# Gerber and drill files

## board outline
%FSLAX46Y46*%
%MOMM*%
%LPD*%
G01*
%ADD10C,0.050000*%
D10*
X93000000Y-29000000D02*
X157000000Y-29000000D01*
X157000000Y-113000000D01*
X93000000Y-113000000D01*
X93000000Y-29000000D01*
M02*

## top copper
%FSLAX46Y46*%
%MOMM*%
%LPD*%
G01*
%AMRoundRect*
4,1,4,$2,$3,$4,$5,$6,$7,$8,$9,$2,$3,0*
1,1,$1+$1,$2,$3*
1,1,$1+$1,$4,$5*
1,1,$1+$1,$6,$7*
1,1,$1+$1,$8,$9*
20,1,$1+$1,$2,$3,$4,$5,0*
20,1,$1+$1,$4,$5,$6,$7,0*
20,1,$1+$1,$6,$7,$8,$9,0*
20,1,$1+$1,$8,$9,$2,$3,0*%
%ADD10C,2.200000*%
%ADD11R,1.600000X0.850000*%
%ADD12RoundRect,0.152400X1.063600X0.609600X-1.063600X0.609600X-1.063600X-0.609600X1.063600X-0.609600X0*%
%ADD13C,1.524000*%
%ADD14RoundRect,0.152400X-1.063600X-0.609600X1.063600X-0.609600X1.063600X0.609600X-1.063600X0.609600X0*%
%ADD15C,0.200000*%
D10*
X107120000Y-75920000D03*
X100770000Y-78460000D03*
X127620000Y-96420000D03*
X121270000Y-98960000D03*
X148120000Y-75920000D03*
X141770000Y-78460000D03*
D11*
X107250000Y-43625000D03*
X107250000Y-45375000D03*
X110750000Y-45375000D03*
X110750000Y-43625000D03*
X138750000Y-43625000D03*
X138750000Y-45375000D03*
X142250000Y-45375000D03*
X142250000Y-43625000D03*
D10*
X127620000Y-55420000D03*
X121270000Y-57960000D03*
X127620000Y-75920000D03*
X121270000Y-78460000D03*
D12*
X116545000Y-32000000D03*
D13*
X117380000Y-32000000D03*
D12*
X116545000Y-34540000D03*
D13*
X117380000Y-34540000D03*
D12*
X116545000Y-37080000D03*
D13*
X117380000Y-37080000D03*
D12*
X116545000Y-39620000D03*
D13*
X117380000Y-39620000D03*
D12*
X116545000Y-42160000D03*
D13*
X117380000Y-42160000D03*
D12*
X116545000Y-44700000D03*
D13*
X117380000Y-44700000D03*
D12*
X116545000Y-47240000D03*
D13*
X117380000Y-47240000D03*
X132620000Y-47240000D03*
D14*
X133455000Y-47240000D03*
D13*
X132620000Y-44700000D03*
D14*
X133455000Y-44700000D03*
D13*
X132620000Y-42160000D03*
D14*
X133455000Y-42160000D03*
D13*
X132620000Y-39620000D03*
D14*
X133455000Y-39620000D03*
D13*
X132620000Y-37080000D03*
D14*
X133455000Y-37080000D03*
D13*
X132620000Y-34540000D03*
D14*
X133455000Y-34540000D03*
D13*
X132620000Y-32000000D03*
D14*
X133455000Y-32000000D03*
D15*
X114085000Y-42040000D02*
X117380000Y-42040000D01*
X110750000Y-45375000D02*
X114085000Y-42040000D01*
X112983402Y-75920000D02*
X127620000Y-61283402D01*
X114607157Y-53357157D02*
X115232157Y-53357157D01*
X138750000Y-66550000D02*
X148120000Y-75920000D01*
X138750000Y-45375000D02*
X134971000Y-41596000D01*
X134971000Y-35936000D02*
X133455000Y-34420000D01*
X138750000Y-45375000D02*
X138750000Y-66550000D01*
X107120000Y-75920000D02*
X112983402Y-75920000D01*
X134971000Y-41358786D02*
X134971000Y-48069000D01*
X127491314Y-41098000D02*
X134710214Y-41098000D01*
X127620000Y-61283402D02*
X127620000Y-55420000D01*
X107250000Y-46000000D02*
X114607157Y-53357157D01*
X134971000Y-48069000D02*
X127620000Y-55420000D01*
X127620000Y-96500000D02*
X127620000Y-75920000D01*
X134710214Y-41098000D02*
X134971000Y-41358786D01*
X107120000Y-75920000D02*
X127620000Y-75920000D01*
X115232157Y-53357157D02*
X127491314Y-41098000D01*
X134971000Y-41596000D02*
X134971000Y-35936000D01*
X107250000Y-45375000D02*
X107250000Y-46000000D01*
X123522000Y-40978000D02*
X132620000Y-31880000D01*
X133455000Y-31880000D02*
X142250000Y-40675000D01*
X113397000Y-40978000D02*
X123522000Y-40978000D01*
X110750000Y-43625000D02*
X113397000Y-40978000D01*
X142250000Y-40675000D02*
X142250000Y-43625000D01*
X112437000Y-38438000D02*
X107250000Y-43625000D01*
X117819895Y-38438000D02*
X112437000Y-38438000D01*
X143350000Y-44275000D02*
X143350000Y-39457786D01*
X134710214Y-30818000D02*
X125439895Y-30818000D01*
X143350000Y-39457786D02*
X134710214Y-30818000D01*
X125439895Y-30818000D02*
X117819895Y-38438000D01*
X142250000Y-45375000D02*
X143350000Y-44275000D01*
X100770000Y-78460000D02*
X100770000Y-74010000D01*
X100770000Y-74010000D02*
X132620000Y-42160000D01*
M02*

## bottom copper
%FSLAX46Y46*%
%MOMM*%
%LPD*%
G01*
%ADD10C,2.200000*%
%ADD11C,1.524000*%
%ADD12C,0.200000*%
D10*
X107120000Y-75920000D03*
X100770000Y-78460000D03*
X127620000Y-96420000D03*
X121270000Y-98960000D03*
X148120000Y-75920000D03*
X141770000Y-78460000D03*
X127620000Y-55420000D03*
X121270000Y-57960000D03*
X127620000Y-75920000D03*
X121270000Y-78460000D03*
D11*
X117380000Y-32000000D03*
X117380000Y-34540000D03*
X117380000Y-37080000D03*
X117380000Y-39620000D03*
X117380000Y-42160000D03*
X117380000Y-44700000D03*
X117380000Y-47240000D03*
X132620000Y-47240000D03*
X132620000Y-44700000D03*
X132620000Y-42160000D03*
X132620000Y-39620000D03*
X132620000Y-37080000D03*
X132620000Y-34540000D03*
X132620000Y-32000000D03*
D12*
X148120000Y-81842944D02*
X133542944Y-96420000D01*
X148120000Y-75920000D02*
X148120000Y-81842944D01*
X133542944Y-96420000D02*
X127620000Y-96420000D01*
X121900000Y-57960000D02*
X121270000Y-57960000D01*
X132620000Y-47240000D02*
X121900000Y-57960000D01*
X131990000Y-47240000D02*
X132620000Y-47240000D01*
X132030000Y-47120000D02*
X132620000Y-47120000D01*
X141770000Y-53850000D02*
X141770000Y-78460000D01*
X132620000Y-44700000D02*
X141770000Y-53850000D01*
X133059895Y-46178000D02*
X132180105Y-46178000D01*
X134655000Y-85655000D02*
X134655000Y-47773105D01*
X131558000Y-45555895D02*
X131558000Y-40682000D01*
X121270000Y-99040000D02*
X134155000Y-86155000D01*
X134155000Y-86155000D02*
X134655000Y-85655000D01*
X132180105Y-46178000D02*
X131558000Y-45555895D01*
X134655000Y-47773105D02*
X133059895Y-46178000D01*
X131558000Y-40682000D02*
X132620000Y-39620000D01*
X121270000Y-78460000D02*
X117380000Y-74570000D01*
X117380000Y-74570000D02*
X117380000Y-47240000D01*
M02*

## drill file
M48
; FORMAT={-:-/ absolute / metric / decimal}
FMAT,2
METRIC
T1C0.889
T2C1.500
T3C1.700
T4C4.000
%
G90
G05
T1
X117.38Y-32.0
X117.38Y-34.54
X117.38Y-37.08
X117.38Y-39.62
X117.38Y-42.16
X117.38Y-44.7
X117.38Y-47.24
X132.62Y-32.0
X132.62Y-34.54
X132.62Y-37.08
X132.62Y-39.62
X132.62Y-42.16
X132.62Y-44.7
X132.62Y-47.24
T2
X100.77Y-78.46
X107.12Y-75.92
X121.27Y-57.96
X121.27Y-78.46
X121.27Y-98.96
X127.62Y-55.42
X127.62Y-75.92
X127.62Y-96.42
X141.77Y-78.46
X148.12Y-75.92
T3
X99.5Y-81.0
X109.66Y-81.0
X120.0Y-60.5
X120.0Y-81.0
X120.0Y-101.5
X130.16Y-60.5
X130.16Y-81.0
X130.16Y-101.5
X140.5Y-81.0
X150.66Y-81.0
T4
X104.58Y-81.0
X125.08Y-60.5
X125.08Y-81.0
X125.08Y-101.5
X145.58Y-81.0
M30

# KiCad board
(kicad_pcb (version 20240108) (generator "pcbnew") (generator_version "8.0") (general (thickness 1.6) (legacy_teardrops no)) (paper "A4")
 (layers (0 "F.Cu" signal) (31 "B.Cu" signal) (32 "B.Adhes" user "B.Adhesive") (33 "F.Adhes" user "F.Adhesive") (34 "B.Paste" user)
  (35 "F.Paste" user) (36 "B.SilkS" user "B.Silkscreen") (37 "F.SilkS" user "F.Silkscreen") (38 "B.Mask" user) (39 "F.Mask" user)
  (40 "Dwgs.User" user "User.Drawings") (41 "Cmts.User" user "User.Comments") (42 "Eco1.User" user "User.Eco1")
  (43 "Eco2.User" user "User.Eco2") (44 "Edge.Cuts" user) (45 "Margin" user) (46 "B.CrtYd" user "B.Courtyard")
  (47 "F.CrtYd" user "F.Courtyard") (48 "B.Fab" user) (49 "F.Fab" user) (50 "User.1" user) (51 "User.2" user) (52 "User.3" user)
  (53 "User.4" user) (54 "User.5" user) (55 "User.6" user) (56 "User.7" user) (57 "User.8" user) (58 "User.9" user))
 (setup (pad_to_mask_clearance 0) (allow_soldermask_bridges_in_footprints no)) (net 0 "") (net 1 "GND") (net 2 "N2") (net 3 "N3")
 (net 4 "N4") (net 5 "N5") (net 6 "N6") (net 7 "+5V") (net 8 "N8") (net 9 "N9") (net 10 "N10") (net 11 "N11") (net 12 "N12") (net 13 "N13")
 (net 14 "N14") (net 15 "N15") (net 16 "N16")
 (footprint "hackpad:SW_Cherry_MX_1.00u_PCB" (layer "F.Cu") (at 107.12 75.92)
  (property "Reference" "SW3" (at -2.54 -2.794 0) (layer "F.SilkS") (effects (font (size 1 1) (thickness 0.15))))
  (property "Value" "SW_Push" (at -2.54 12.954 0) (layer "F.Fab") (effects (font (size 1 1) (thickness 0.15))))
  (pad "" np_thru_hole circle (at -7.62 5.08) (size 1.7 1.7) (drill 1.7) (layers "*.Cu" "*.Mask"))
  (pad "" np_thru_hole circle (at -2.54 5.08) (size 4 4) (drill 4) (layers "*.Cu" "*.Mask"))
  (pad "" np_thru_hole circle (at 2.54 5.08) (size 1.7 1.7) (drill 1.7) (layers "*.Cu" "*.Mask"))
  (pad "1" thru_hole circle (at 0 0) (size 2.2 2.2) (drill 1.5) (layers "*.Cu" "*.Mask") (remove_unused_layers no) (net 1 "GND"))
  (pad "2" thru_hole circle (at -6.35 2.54) (size 2.2 2.2) (drill 1.5) (layers "*.Cu" "*.Mask") (remove_unused_layers no) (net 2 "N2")))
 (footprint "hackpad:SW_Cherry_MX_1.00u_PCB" (layer "F.Cu") (at 127.62 96.42)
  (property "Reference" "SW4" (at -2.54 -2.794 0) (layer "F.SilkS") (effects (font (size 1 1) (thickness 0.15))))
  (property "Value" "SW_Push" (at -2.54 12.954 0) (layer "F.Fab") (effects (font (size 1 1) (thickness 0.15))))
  (pad "" np_thru_hole circle (at -7.62 5.08) (size 1.7 1.7) (drill 1.7) (layers "*.Cu" "*.Mask"))
  (pad "" np_thru_hole circle (at -2.54 5.08) (size 4 4) (drill 4) (layers "*.Cu" "*.Mask"))
  (pad "" np_thru_hole circle (at 2.54 5.08) (size 1.7 1.7) (drill 1.7) (layers "*.Cu" "*.Mask"))
  (pad "1" thru_hole circle (at 0 0) (size 2.2 2.2) (drill 1.5) (layers "*.Cu" "*.Mask") (remove_unused_layers no) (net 1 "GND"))
  (pad "2" thru_hole circle (at -6.35 2.54) (size 2.2 2.2) (drill 1.5) (layers "*.Cu" "*.Mask") (remove_unused_layers no) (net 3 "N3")))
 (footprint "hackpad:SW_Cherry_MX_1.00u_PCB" (layer "F.Cu") (at 148.12 75.92)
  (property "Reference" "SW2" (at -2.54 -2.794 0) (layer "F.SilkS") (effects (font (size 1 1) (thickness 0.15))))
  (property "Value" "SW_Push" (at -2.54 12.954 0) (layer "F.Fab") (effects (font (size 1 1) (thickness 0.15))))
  (pad "" np_thru_hole circle (at -7.62 5.08) (size 1.7 1.7) (drill 1.7) (layers "*.Cu" "*.Mask"))
  (pad "" np_thru_hole circle (at -2.54 5.08) (size 4 4) (drill 4) (layers "*.Cu" "*.Mask"))
  (pad "" np_thru_hole circle (at 2.54 5.08) (size 1.7 1.7) (drill 1.7) (layers "*.Cu" "*.Mask"))
  (pad "1" thru_hole circle (at 0 0) (size 2.2 2.2) (drill 1.5) (layers "*.Cu" "*.Mask") (remove_unused_layers no) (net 1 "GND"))
  (pad "2" thru_hole circle (at -6.35 2.54) (size 2.2 2.2) (drill 1.5) (layers "*.Cu" "*.Mask") (remove_unused_layers no) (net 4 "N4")))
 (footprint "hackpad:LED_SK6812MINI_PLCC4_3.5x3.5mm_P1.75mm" (layer "F.Cu") (at 109 44.5)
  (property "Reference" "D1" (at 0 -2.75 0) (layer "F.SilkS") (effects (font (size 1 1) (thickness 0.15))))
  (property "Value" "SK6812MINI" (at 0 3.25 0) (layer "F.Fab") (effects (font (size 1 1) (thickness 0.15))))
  (pad "1" smd rect (at -1.75 -0.875) (size 1.6 0.85) (layers "F.Cu" "F.Paste" "F.Mask") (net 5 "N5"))
  (pad "2" smd rect (at -1.75 0.875) (size 1.6 0.85) (layers "F.Cu" "F.Paste" "F.Mask") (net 1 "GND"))
  (pad "3" smd rect (at 1.75 0.875) (size 1.6 0.85) (layers "F.Cu" "F.Paste" "F.Mask") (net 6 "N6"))
  (pad "4" smd rect (at 1.75 -0.875) (size 1.6 0.85) (layers "F.Cu" "F.Paste" "F.Mask") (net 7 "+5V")))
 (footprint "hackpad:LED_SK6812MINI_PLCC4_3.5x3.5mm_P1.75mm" (layer "F.Cu") (at 140.5 44.5)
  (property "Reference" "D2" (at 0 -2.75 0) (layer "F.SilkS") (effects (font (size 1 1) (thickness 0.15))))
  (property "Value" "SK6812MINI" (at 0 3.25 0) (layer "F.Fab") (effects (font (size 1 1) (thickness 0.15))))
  (pad "1" smd rect (at -1.75 -0.875) (size 1.6 0.85) (layers "F.Cu" "F.Paste" "F.Mask") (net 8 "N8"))
  (pad "2" smd rect (at -1.75 0.875) (size 1.6 0.85) (layers "F.Cu" "F.Paste" "F.Mask") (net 1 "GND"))
  (pad "3" smd rect (at 1.75 0.875) (size 1.6 0.85) (layers "F.Cu" "F.Paste" "F.Mask") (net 5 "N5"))
  (pad "4" smd rect (at 1.75 -0.875) (size 1.6 0.85) (layers "F.Cu" "F.Paste" "F.Mask") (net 7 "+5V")))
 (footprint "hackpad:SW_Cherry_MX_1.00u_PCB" (layer "F.Cu") (at 127.62 55.42)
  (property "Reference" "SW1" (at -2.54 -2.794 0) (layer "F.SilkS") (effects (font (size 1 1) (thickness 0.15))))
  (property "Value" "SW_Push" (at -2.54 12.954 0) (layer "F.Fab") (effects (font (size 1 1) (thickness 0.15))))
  (pad "" np_thru_hole circle (at -7.62 5.08) (size 1.7 1.7) (drill 1.7) (layers "*.Cu" "*.Mask"))
  (pad "" np_thru_hole circle (at -2.54 5.08) (size 4 4) (drill 4) (layers "*.Cu" "*.Mask"))
  (pad "" np_thru_hole circle (at 2.54 5.08) (size 1.7 1.7) (drill 1.7) (layers "*.Cu" "*.Mask"))
  (pad "1" thru_hole circle (at 0 0) (size 2.2 2.2) (drill 1.5) (layers "*.Cu" "*.Mask") (remove_unused_layers no) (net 1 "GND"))
  (pad "2" thru_hole circle (at -6.35 2.54) (size 2.2 2.2) (drill 1.5) (layers "*.Cu" "*.Mask") (remove_unused_layers no) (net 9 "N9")))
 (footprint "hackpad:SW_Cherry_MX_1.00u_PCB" (layer "F.Cu") (at 127.62 75.92)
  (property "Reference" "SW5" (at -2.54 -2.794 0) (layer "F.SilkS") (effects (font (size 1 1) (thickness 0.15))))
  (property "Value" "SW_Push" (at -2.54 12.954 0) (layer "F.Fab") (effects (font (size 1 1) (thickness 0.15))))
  (pad "" np_thru_hole circle (at -7.62 5.08) (size 1.7 1.7) (drill 1.7) (layers "*.Cu" "*.Mask"))
  (pad "" np_thru_hole circle (at -2.54 5.08) (size 4 4) (drill 4) (layers "*.Cu" "*.Mask"))
  (pad "" np_thru_hole circle (at 2.54 5.08) (size 1.7 1.7) (drill 1.7) (layers "*.Cu" "*.Mask"))
  (pad "1" thru_hole circle (at 0 0) (size 2.2 2.2) (drill 1.5) (layers "*.Cu" "*.Mask") (remove_unused_layers no) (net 1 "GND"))
  (pad "2" thru_hole circle (at -6.35 2.54) (size 2.2 2.2) (drill 1.5) (layers "*.Cu" "*.Mask") (remove_unused_layers no) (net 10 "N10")))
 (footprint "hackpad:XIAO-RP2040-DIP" (layer "F.Cu") (at 125 39.62)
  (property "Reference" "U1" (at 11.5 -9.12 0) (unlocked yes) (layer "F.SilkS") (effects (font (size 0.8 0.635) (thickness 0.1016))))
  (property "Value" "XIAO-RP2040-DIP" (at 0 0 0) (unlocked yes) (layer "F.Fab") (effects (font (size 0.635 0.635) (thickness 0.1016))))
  (pad "1" smd roundrect (at -8.455 -7.62 180) (size 2.432 1.524) (layers "F.Cu" "F.Mask") (roundrect_rratio 0.1) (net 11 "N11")
   (thermal_bridge_angle 45))
  (pad "1" thru_hole circle (at -7.62 -7.62 180) (size 1.524 1.524) (drill 0.889) (layers "*.Cu" "*.Mask") (remove_unused_layers no)
   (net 11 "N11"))
  (pad "2" smd roundrect (at -8.455 -5.08 180) (size 2.432 1.524) (layers "F.Cu" "F.Mask") (roundrect_rratio 0.1) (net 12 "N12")
   (thermal_bridge_angle 45))
  (pad "2" thru_hole circle (at -7.62 -5.08 180) (size 1.524 1.524) (drill 0.889) (layers "*.Cu" "*.Mask") (remove_unused_layers no)
   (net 12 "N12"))
  (pad "3" smd roundrect (at -8.455 -2.54 180) (size 2.432 1.524) (layers "F.Cu" "F.Mask") (roundrect_rratio 0.1) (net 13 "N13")
   (thermal_bridge_angle 45))
  (pad "3" thru_hole circle (at -7.62 -2.54 180) (size 1.524 1.524) (drill 0.889) (layers "*.Cu" "*.Mask") (remove_unused_layers no)
   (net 13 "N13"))
  (pad "4" smd roundrect (at -8.455 0 180) (size 2.432 1.524) (layers "F.Cu" "F.Mask") (roundrect_rratio 0.1) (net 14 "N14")
   (thermal_bridge_angle 45))
  (pad "4" thru_hole circle (at -7.62 0 180) (size 1.524 1.524) (drill 0.889) (layers "*.Cu" "*.Mask") (remove_unused_layers no)
   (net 14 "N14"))
  (pad "5" smd roundrect (at -8.455 2.54 180) (size 2.432 1.524) (layers "F.Cu" "F.Mask") (roundrect_rratio 0.1) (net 6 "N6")
   (thermal_bridge_angle 45))
  (pad "5" thru_hole circle (at -7.62 2.54 180) (size 1.524 1.524) (drill 0.889) (layers "*.Cu" "*.Mask") (remove_unused_layers no)
   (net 6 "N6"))
  (pad "6" smd roundrect (at -8.455 5.08 180) (size 2.432 1.524) (layers "F.Cu" "F.Mask") (roundrect_rratio 0.1) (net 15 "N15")
   (thermal_bridge_angle 45))
  (pad "6" thru_hole circle (at -7.62 5.08 180) (size 1.524 1.524) (drill 0.889) (layers "*.Cu" "*.Mask") (remove_unused_layers no)
   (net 15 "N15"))
  (pad "7" smd roundrect (at -8.455 7.62 180) (size 2.432 1.524) (layers "F.Cu" "F.Mask") (roundrect_rratio 0.1) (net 10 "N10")
   (thermal_bridge_angle 45))
  (pad "7" thru_hole circle (at -7.62 7.62 180) (size 1.524 1.524) (drill 0.889) (layers "*.Cu" "*.Mask") (remove_unused_layers no)
   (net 10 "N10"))
  (pad "8" thru_hole circle (at 7.62 7.62) (size 1.524 1.524) (drill 0.889) (layers "*.Cu" "*.Mask") (remove_unused_layers no) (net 9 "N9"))
  (pad "8" smd roundrect (at 8.455 7.62) (size 2.432 1.524) (layers "F.Cu" "F.Mask") (roundrect_rratio 0.1) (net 9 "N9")
   (thermal_bridge_angle 45))
  (pad "9" thru_hole circle (at 7.62 5.08) (size 1.524 1.524) (drill 0.889) (layers "*.Cu" "*.Mask") (remove_unused_layers no) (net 4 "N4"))
  (pad "9" smd roundrect (at 8.455 5.08) (size 2.432 1.524) (layers "F.Cu" "F.Mask") (roundrect_rratio 0.1) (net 4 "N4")
   (thermal_bridge_angle 45))
  (pad "10" thru_hole circle (at 7.62 2.54) (size 1.524 1.524) (drill 0.889) (layers "*.Cu" "*.Mask") (remove_unused_layers no) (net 2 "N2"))
  (pad "10" smd roundrect (at 8.455 2.54) (size 2.432 1.524) (layers "F.Cu" "F.Mask") (roundrect_rratio 0.1) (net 2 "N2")
   (thermal_bridge_angle 45))
  (pad "11" thru_hole circle (at 7.62 0) (size 1.524 1.524) (drill 0.889) (layers "*.Cu" "*.Mask") (remove_unused_layers no) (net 3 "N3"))
  (pad "11" smd roundrect (at 8.455 0) (size 2.432 1.524) (layers "F.Cu" "F.Mask") (roundrect_rratio 0.1) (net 3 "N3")
   (thermal_bridge_angle 45))
  (pad "12" thru_hole circle (at 7.62 -2.54) (size 1.524 1.524) (drill 0.889) (layers "*.Cu" "*.Mask") (remove_unused_layers no)
   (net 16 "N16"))
  (pad "12" smd roundrect (at 8.455 -2.54) (size 2.432 1.524) (layers "F.Cu" "F.Mask") (roundrect_rratio 0.1) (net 16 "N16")
   (thermal_bridge_angle 45))
  (pad "13" thru_hole circle (at 7.62 -5.08) (size 1.524 1.524) (drill 0.889) (layers "*.Cu" "*.Mask") (remove_unused_layers no)
   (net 1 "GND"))
  (pad "13" smd roundrect (at 8.455 -5.08) (size 2.432 1.524) (layers "F.Cu" "F.Mask") (roundrect_rratio 0.1) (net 1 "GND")
   (thermal_bridge_angle 45))
  (pad "14" thru_hole circle (at 7.62 -7.62) (size 1.524 1.524) (drill 0.889) (layers "*.Cu" "*.Mask") (remove_unused_layers no)
   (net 7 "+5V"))
  (pad "14" smd roundrect (at 8.455 -7.62) (size 2.432 1.524) (layers "F.Cu" "F.Mask") (roundrect_rratio 0.1) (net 7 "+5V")
   (thermal_bridge_angle 45)))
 (gr_rect (start 93 29) (end 157 113) (stroke (width 0.05) (type default)) (fill none) (layer "Edge.Cuts"))
 (segment (start 114.085 42.04) (end 117.38 42.04) (width 0.2) (layer "F.Cu") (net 6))
 (segment (start 110.75 45.375) (end 114.085 42.04) (width 0.2) (layer "F.Cu") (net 6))
 (segment (start 112.983402 75.92) (end 127.62 61.283402) (width 0.2) (layer "F.Cu") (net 1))
 (segment (start 114.607157 53.357157) (end 115.232157 53.357157) (width 0.2) (layer "F.Cu") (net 1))
 (segment (start 138.75 66.55) (end 148.12 75.92) (width 0.2) (layer "F.Cu") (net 1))
 (segment (start 138.75 45.375) (end 134.971 41.596) (width 0.2) (layer "F.Cu") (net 1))
 (segment (start 134.971 35.936) (end 133.455 34.42) (width 0.2) (layer "F.Cu") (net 1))
 (segment (start 138.75 45.375) (end 138.75 66.55) (width 0.2) (layer "F.Cu") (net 1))
 (segment (start 107.12 75.92) (end 112.983402 75.92) (width 0.2) (layer "F.Cu") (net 1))
 (segment (start 134.971 41.358786) (end 134.971 48.069) (width 0.2) (layer "F.Cu") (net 1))
 (segment (start 127.491314 41.098) (end 134.710214 41.098) (width 0.2) (layer "F.Cu") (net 1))
 (segment (start 127.62 61.283402) (end 127.62 55.42) (width 0.2) (layer "F.Cu") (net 1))
 (segment (start 107.25 46) (end 114.607157 53.357157) (width 0.2) (layer "F.Cu") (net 1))
 (segment (start 134.971 48.069) (end 127.62 55.42) (width 0.2) (layer "F.Cu") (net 1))
 (segment (start 127.62 96.5) (end 127.62 75.92) (width 0.2) (layer "F.Cu") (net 1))
 (segment (start 134.710214 41.098) (end 134.971 41.358786) (width 0.2) (layer "F.Cu") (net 1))
 (segment (start 107.12 75.92) (end 127.62 75.92) (width 0.2) (layer "F.Cu") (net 1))
 (segment (start 115.232157 53.357157) (end 127.491314 41.098) (width 0.2) (layer "F.Cu") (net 1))
 (segment (start 134.971 41.596) (end 134.971 35.936) (width 0.2) (layer "F.Cu") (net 1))
 (segment (start 107.25 45.375) (end 107.25 46) (width 0.2) (layer "F.Cu") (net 1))
 (segment (start 148.12 81.842944) (end 133.542944 96.42) (width 0.2) (layer "B.Cu") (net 1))
 (segment (start 148.12 75.92) (end 148.12 81.842944) (width 0.2) (layer "B.Cu") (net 1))
 (segment (start 133.542944 96.42) (end 127.62 96.42) (width 0.2) (layer "B.Cu") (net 1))
 (segment (start 123.522 40.978) (end 132.62 31.88) (width 0.2) (layer "F.Cu") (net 7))
 (segment (start 133.455 31.88) (end 142.25 40.675) (width 0.2) (layer "F.Cu") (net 7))
 (segment (start 113.397 40.978) (end 123.522 40.978) (width 0.2) (layer "F.Cu") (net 7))
 (segment (start 110.75 43.625) (end 113.397 40.978) (width 0.2) (layer "F.Cu") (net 7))
 (segment (start 142.25 40.675) (end 142.25 43.625) (width 0.2) (layer "F.Cu") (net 7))
 (segment (start 112.437 38.438) (end 107.25 43.625) (width 0.2) (layer "F.Cu") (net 5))
 (segment (start 117.819895 38.438) (end 112.437 38.438) (width 0.2) (layer "F.Cu") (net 5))
 (segment (start 143.35 44.275) (end 143.35 39.457786) (width 0.2) (layer "F.Cu") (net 5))
 (segment (start 134.710214 30.818) (end 125.439895 30.818) (width 0.2) (layer "F.Cu") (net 5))
 (segment (start 143.35 39.457786) (end 134.710214 30.818) (width 0.2) (layer "F.Cu") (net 5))
 (segment (start 125.439895 30.818) (end 117.819895 38.438) (width 0.2) (layer "F.Cu") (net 5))
 (segment (start 142.25 45.375) (end 143.35 44.275) (width 0.2) (layer "F.Cu") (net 5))
 (segment (start 121.9 57.96) (end 121.27 57.96) (width 0.2) (layer "B.Cu") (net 9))
 (segment (start 132.62 47.24) (end 121.9 57.96) (width 0.2) (layer "B.Cu") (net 9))
 (segment (start 131.99 47.24) (end 132.62 47.24) (width 0.2) (layer "B.Cu") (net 9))
 (segment (start 132.03 47.12) (end 132.62 47.12) (width 0.2) (layer "B.Cu") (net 9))
 (segment (start 141.77 53.85) (end 141.77 78.46) (width 0.2) (layer "B.Cu") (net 4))
 (segment (start 132.62 44.7) (end 141.77 53.85) (width 0.2) (layer "B.Cu") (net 4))
 (segment (start 100.77 78.46) (end 100.77 74.01) (width 0.2) (layer "F.Cu") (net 2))
 (segment (start 100.77 74.01) (end 132.62 42.16) (width 0.2) (layer "F.Cu") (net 2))
 (segment (start 133.059895 46.178) (end 132.180105 46.178) (width 0.2) (layer "B.Cu") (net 3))
 (segment (start 134.655 85.655) (end 134.655 47.773105) (width 0.2) (layer "B.Cu") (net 3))
 (segment (start 131.558 45.555895) (end 131.558 40.682) (width 0.2) (layer "B.Cu") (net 3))
 (segment (start 121.27 99.04) (end 134.155 86.155) (width 0.2) (layer "B.Cu") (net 3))
 (segment (start 134.155 86.155) (end 134.655 85.655) (width 0.2) (layer "B.Cu") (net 3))
 (segment (start 132.180105 46.178) (end 131.558 45.555895) (width 0.2) (layer "B.Cu") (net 3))
 (segment (start 134.655 47.773105) (end 133.059895 46.178) (width 0.2) (layer "B.Cu") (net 3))
 (segment (start 131.558 40.682) (end 132.62 39.62) (width 0.2) (layer "B.Cu") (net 3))
 (segment (start 121.27 78.46) (end 117.38 74.57) (width 0.2) (layer "B.Cu") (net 10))
 (segment (start 117.38 74.57) (end 117.38 47.24) (width 0.2) (layer "B.Cu") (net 10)))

